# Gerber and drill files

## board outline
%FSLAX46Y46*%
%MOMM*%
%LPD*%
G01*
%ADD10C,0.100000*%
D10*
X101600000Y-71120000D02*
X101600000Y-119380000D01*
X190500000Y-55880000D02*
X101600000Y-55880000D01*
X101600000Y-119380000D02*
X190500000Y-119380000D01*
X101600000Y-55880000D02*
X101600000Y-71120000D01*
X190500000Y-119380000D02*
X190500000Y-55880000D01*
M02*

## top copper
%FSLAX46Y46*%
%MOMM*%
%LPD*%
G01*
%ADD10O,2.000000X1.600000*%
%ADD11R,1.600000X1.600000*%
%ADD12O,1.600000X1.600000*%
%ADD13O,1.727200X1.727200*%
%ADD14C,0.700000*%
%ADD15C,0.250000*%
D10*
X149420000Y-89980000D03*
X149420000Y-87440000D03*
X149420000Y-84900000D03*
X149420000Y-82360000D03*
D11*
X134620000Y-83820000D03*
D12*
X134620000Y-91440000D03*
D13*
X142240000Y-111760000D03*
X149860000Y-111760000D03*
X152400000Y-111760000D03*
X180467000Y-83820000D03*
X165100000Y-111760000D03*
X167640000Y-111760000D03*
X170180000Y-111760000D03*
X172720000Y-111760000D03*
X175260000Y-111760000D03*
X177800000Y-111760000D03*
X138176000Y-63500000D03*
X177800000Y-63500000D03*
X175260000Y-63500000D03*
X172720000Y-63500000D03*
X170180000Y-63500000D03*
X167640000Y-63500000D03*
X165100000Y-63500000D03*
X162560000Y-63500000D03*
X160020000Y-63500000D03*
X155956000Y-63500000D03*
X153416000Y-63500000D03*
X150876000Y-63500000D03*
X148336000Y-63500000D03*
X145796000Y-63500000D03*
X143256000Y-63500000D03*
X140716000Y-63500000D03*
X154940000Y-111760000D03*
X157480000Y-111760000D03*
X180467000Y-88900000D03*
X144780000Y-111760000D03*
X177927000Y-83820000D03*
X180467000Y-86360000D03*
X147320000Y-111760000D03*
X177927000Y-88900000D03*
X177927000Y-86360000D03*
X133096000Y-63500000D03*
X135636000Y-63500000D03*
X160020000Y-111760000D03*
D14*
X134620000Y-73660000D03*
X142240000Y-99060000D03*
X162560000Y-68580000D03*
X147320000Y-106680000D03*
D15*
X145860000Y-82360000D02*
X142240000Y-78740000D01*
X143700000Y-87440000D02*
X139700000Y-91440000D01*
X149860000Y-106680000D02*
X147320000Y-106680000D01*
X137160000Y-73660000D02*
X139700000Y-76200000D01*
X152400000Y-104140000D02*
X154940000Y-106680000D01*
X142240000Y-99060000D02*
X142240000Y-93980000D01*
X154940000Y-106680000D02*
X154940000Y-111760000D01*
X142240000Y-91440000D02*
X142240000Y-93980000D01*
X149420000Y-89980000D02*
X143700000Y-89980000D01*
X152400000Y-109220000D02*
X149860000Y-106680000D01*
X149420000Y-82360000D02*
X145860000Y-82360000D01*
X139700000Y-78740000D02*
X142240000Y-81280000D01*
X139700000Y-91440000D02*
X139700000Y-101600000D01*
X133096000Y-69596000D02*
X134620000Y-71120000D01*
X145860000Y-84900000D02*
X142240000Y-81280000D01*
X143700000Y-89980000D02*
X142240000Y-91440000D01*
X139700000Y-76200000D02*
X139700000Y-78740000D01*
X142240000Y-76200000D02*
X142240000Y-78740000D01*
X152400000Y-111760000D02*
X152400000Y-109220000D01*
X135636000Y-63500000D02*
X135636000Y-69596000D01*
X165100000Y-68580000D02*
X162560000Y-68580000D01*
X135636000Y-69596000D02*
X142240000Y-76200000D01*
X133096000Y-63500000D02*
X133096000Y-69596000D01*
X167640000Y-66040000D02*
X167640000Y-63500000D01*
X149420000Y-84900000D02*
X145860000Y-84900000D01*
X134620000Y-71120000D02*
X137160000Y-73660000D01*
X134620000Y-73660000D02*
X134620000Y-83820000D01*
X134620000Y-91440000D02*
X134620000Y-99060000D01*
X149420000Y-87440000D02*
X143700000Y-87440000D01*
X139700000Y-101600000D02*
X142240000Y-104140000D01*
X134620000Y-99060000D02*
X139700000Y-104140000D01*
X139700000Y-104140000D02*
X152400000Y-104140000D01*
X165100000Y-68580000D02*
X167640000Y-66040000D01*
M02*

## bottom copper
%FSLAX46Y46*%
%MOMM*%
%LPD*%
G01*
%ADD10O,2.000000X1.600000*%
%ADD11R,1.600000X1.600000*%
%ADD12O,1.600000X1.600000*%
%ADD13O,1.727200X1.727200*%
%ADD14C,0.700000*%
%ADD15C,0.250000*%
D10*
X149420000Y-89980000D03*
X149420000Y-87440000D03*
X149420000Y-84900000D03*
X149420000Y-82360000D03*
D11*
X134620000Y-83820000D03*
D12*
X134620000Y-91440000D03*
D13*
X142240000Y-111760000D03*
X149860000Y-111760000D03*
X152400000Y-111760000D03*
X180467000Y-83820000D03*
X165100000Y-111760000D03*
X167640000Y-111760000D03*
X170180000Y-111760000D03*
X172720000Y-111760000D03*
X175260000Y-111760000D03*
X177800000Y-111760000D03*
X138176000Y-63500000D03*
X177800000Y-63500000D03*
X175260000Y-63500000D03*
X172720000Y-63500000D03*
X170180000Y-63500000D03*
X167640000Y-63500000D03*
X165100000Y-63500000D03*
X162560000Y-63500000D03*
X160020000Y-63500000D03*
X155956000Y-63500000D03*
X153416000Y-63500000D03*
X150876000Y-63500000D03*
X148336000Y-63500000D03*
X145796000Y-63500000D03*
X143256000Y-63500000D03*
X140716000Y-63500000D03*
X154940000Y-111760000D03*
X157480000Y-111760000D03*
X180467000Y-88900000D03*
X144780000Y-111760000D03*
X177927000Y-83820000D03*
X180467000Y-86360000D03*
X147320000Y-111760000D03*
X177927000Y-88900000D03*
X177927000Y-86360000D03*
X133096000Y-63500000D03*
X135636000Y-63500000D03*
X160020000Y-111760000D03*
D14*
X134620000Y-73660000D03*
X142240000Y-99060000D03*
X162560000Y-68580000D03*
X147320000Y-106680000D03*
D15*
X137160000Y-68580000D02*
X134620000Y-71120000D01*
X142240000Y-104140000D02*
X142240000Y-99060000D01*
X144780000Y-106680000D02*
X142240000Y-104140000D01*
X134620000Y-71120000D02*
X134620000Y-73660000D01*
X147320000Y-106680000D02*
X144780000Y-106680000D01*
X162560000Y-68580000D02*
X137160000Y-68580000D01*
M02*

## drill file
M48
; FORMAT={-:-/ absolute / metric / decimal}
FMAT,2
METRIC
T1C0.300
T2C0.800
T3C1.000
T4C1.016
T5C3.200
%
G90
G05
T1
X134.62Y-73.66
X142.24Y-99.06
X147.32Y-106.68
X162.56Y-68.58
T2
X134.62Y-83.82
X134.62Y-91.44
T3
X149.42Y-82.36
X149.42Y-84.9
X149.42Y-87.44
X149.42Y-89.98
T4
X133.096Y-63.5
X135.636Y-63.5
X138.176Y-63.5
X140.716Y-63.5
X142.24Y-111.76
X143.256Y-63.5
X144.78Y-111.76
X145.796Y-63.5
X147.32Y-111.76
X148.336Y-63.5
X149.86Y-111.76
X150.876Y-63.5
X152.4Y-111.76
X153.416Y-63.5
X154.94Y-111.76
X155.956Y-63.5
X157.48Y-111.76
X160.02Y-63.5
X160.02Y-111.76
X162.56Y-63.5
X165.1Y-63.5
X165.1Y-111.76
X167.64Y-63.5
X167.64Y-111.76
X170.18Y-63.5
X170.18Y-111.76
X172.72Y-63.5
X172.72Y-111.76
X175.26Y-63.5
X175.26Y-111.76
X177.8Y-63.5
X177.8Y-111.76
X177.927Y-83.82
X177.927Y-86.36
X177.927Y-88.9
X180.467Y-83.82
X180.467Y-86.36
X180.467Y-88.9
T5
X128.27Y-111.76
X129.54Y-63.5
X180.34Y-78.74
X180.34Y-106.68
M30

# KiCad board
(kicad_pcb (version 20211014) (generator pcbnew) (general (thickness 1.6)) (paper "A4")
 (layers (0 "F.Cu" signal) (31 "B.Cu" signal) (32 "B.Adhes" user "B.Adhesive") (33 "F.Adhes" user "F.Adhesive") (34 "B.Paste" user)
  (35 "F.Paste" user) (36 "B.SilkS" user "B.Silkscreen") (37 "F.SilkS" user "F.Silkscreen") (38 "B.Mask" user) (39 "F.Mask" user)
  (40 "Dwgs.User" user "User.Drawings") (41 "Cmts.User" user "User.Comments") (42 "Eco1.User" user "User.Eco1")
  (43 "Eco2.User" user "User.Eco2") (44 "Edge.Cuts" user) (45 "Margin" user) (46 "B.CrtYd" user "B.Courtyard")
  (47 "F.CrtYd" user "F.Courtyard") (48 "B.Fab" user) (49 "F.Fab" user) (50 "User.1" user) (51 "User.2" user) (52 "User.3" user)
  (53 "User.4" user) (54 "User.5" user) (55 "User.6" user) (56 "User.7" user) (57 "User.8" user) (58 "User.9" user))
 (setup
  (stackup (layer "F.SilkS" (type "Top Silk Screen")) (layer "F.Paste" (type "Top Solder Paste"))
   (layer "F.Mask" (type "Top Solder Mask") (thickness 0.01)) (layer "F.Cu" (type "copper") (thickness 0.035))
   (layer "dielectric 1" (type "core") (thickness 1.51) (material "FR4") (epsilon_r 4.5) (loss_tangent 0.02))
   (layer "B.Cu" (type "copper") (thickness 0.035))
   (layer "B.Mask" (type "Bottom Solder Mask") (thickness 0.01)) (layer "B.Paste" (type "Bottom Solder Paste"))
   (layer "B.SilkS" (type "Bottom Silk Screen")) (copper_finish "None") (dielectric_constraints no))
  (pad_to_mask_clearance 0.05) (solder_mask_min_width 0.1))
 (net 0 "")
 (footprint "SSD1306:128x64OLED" (layer "F.Cu") (at 160.02 86.36 90)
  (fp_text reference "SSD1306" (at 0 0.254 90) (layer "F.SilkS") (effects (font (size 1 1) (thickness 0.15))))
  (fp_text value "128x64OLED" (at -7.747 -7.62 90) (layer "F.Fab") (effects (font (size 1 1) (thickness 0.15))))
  (pad "1" thru_hole oval locked (at -3.62 -10.6 180) (size 2 1.6) (drill 1) (layers *.Cu *.Mask))
  (pad "2" thru_hole oval locked (at -1.08 -10.6 180) (size 2 1.6) (drill 1) (layers *.Cu *.Mask))
  (pad "3" thru_hole oval locked (at 1.46 -10.6 180) (size 2 1.6) (drill 1) (layers *.Cu *.Mask))
  (pad "4" thru_hole oval locked (at 4 -10.6 180) (size 2 1.6) (drill 1) (layers *.Cu *.Mask)))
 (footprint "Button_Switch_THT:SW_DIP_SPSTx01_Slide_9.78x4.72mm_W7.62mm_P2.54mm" (layer "F.Cu") (at 134.62 83.82 -90)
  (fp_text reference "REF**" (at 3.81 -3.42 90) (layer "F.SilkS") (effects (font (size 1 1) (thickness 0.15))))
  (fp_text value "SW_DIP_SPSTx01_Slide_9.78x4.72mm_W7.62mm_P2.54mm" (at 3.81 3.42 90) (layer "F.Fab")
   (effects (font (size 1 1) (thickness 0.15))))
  (pad "1" thru_hole rect (at 0 0 270) (size 1.6 1.6) (drill 0.8) (layers *.Cu *.Mask))
  (pad "2" thru_hole oval (at 7.62 0 270) (size 1.6 1.6) (drill 0.8) (layers *.Cu *.Mask)))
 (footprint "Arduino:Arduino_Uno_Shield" (layer "F.Cu") (at 114.3 114.3)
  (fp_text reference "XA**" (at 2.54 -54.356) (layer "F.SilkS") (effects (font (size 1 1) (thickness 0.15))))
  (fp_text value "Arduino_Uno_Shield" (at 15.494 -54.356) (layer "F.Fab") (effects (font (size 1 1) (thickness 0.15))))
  (pad "" np_thru_hole circle (at 66.04 -35.56) (size 3.2 3.2) (drill 3.2) (layers *.Cu *.Mask))
  (pad "" np_thru_hole circle (at 66.04 -7.62) (size 3.2 3.2) (drill 3.2) (layers *.Cu *.Mask))
  (pad "" np_thru_hole circle (at 13.97 -2.54) (size 3.2 3.2) (drill 3.2) (layers *.Cu *.Mask))
  (pad "" thru_hole oval (at 27.94 -2.54) (size 1.7272 1.7272) (drill 1.016) (layers *.Cu *.Mask))
  (pad "" np_thru_hole circle (at 15.24 -50.8) (size 3.2 3.2) (drill 3.2) (layers *.Cu *.Mask))
  (pad "3V3" thru_hole oval (at 35.56 -2.54) (size 1.7272 1.7272) (drill 1.016) (layers *.Cu *.Mask))
  (pad "5V1" thru_hole oval (at 38.1 -2.54) (size 1.7272 1.7272) (drill 1.016) (layers *.Cu *.Mask))
  (pad "5V2" thru_hole oval (at 66.167 -30.48) (size 1.7272 1.7272) (drill 1.016) (layers *.Cu *.Mask))
  (pad "A0" thru_hole oval (at 50.8 -2.54) (size 1.7272 1.7272) (drill 1.016) (layers *.Cu *.Mask))
  (pad "A1" thru_hole oval (at 53.34 -2.54) (size 1.7272 1.7272) (drill 1.016) (layers *.Cu *.Mask))
  (pad "A2" thru_hole oval (at 55.88 -2.54) (size 1.7272 1.7272) (drill 1.016) (layers *.Cu *.Mask))
  (pad "A3" thru_hole oval (at 58.42 -2.54) (size 1.7272 1.7272) (drill 1.016) (layers *.Cu *.Mask))
  (pad "A4" thru_hole oval (at 60.96 -2.54) (size 1.7272 1.7272) (drill 1.016) (layers *.Cu *.Mask))
  (pad "A5" thru_hole oval (at 63.5 -2.54) (size 1.7272 1.7272) (drill 1.016) (layers *.Cu *.Mask))
  (pad "AREF" thru_hole oval (at 23.876 -50.8) (size 1.7272 1.7272) (drill 1.016) (layers *.Cu *.Mask))
  (pad "D0" thru_hole oval (at 63.5 -50.8) (size 1.7272 1.7272) (drill 1.016) (layers *.Cu *.Mask))
  (pad "D1" thru_hole oval (at 60.96 -50.8) (size 1.7272 1.7272) (drill 1.016) (layers *.Cu *.Mask))
  (pad "D2" thru_hole oval (at 58.42 -50.8) (size 1.7272 1.7272) (drill 1.016) (layers *.Cu *.Mask))
  (pad "D3" thru_hole oval (at 55.88 -50.8) (size 1.7272 1.7272) (drill 1.016) (layers *.Cu *.Mask))
  (pad "D4" thru_hole oval (at 53.34 -50.8) (size 1.7272 1.7272) (drill 1.016) (layers *.Cu *.Mask))
  (pad "D5" thru_hole oval (at 50.8 -50.8) (size 1.7272 1.7272) (drill 1.016) (layers *.Cu *.Mask))
  (pad "D6" thru_hole oval (at 48.26 -50.8) (size 1.7272 1.7272) (drill 1.016) (layers *.Cu *.Mask))
  (pad "D7" thru_hole oval (at 45.72 -50.8) (size 1.7272 1.7272) (drill 1.016) (layers *.Cu *.Mask))
  (pad "D8" thru_hole oval (at 41.656 -50.8) (size 1.7272 1.7272) (drill 1.016) (layers *.Cu *.Mask))
  (pad "D9" thru_hole oval (at 39.116 -50.8) (size 1.7272 1.7272) (drill 1.016) (layers *.Cu *.Mask))
  (pad "D10" thru_hole oval (at 36.576 -50.8) (size 1.7272 1.7272) (drill 1.016) (layers *.Cu *.Mask))
  (pad "D11" thru_hole oval (at 34.036 -50.8) (size 1.7272 1.7272) (drill 1.016) (layers *.Cu *.Mask))
  (pad "D12" thru_hole oval (at 31.496 -50.8) (size 1.7272 1.7272) (drill 1.016) (layers *.Cu *.Mask))
  (pad "D13" thru_hole oval (at 28.956 -50.8) (size 1.7272 1.7272) (drill 1.016) (layers *.Cu *.Mask))
  (pad "GND1" thru_hole oval (at 26.416 -50.8) (size 1.7272 1.7272) (drill 1.016) (layers *.Cu *.Mask))
  (pad "GND2" thru_hole oval (at 40.64 -2.54) (size 1.7272 1.7272) (drill 1.016) (layers *.Cu *.Mask))
  (pad "GND3" thru_hole oval (at 43.18 -2.54) (size 1.7272 1.7272) (drill 1.016) (layers *.Cu *.Mask))
  (pad "GND4" thru_hole oval (at 66.167 -25.4) (size 1.7272 1.7272) (drill 1.016) (layers *.Cu *.Mask))
  (pad "IORF" thru_hole oval (at 30.48 -2.54) (size 1.7272 1.7272) (drill 1.016) (layers *.Cu *.Mask))
  (pad "MISO" thru_hole oval (at 63.627 -30.48) (size 1.7272 1.7272) (drill 1.016) (layers *.Cu *.Mask))
  (pad "MOSI" thru_hole oval (at 66.167 -27.94) (size 1.7272 1.7272) (drill 1.016) (layers *.Cu *.Mask))
  (pad "RST1" thru_hole oval (at 33.02 -2.54) (size 1.7272 1.7272) (drill 1.016) (layers *.Cu *.Mask))
  (pad "RST2" thru_hole oval (at 63.627 -25.4) (size 1.7272 1.7272) (drill 1.016) (layers *.Cu *.Mask))
  (pad "SCK" thru_hole oval (at 63.627 -27.94) (size 1.7272 1.7272) (drill 1.016) (layers *.Cu *.Mask))
  (pad "SCL" thru_hole oval (at 18.796 -50.8) (size 1.7272 1.7272) (drill 1.016) (layers *.Cu *.Mask))
  (pad "SDA" thru_hole oval (at 21.336 -50.8) (size 1.7272 1.7272) (drill 1.016) (layers *.Cu *.Mask))
  (pad "VIN" thru_hole oval (at 45.72 -2.54) (size 1.7272 1.7272) (drill 1.016) (layers *.Cu *.Mask)))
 (gr_line (start 101.6 71.12) (end 101.6 119.38) (layer "Edge.Cuts") (width 0.1))
 (gr_line (start 190.5 55.88) (end 101.6 55.88) (layer "Edge.Cuts") (width 0.1))
 (gr_line (start 101.6 119.38) (end 190.5 119.38) (layer "Edge.Cuts") (width 0.1))
 (gr_line (start 101.6 55.88) (end 101.6 71.12) (layer "Edge.Cuts") (width 0.1))
 (gr_line (start 190.5 119.38) (end 190.5 55.88) (layer "Edge.Cuts") (width 0.1))
 (segment (start 145.86 82.36) (end 142.24 78.74) (width 0.25) (layer "F.Cu") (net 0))
 (segment (start 143.7 87.44) (end 139.7 91.44) (width 0.25) (layer "F.Cu") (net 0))
 (segment (start 149.86 106.68) (end 147.32 106.68) (width 0.25) (layer "F.Cu") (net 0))
 (segment (start 137.16 73.66) (end 139.7 76.2) (width 0.25) (layer "F.Cu") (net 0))
 (segment (start 152.4 104.14) (end 154.94 106.68) (width 0.25) (layer "F.Cu") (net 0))
 (segment (start 142.24 99.06) (end 142.24 93.98) (width 0.25) (layer "F.Cu") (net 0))
 (segment (start 154.94 106.68) (end 154.94 111.76) (width 0.25) (layer "F.Cu") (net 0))
 (segment (start 142.24 91.44) (end 142.24 93.98) (width 0.25) (layer "F.Cu") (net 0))
 (segment (start 149.42 89.98) (end 143.7 89.98) (width 0.25) (layer "F.Cu") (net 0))
 (segment (start 152.4 109.22) (end 149.86 106.68) (width 0.25) (layer "F.Cu") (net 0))
 (segment (start 149.42 82.36) (end 145.86 82.36) (width 0.25) (layer "F.Cu") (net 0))
 (segment (start 139.7 78.74) (end 142.24 81.28) (width 0.25) (layer "F.Cu") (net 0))
 (segment (start 139.7 91.44) (end 139.7 101.6) (width 0.25) (layer "F.Cu") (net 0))
 (segment (start 133.096 69.596) (end 134.62 71.12) (width 0.25) (layer "F.Cu") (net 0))
 (segment (start 145.86 84.9) (end 142.24 81.28) (width 0.25) (layer "F.Cu") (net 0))
 (segment (start 143.7 89.98) (end 142.24 91.44) (width 0.25) (layer "F.Cu") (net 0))
 (segment (start 139.7 76.2) (end 139.7 78.74) (width 0.25) (layer "F.Cu") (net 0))
 (segment (start 142.24 76.2) (end 142.24 78.74) (width 0.25) (layer "F.Cu") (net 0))
 (segment (start 152.4 111.76) (end 152.4 109.22) (width 0.25) (layer "F.Cu") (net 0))
 (segment (start 135.636 63.5) (end 135.636 69.596) (width 0.25) (layer "F.Cu") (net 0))
 (segment (start 165.1 68.58) (end 162.56 68.58) (width 0.25) (layer "F.Cu") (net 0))
 (segment (start 135.636 69.596) (end 142.24 76.2) (width 0.25) (layer "F.Cu") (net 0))
 (segment (start 133.096 63.5) (end 133.096 69.596) (width 0.25) (layer "F.Cu") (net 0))
 (segment (start 167.64 66.04) (end 167.64 63.5) (width 0.25) (layer "F.Cu") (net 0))
 (segment (start 149.42 84.9) (end 145.86 84.9) (width 0.25) (layer "F.Cu") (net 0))
 (segment (start 134.62 71.12) (end 137.16 73.66) (width 0.25) (layer "F.Cu") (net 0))
 (segment (start 134.62 73.66) (end 134.62 83.82) (width 0.25) (layer "F.Cu") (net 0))
 (segment (start 134.62 91.44) (end 134.62 99.06) (width 0.25) (layer "F.Cu") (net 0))
 (segment (start 149.42 87.44) (end 143.7 87.44) (width 0.25) (layer "F.Cu") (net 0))
 (segment (start 139.7 101.6) (end 142.24 104.14) (width 0.25) (layer "F.Cu") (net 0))
 (segment (start 134.62 99.06) (end 139.7 104.14) (width 0.25) (layer "F.Cu") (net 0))
 (segment (start 139.7 104.14) (end 152.4 104.14) (width 0.25) (layer "F.Cu") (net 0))
 (segment (start 165.1 68.58) (end 167.64 66.04) (width 0.25) (layer "F.Cu") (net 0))
 (via (at 134.62 73.66) (size 0.7) (drill 0.3) (layers "F.Cu" "B.Cu") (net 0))
 (via (at 142.24 99.06) (size 0.7) (drill 0.3) (layers "F.Cu" "B.Cu") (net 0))
 (via (at 162.56 68.58) (size 0.7) (drill 0.3) (layers "F.Cu" "B.Cu") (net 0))
 (via (at 147.32 106.68) (size 0.7) (drill 0.3) (layers "F.Cu" "B.Cu") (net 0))
 (segment (start 137.16 68.58) (end 134.62 71.12) (width 0.25) (layer "B.Cu") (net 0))
 (segment (start 142.24 104.14) (end 142.24 99.06) (width 0.25) (layer "B.Cu") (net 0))
 (segment (start 144.78 106.68) (end 142.24 104.14) (width 0.25) (layer "B.Cu") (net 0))
 (segment (start 134.62 71.12) (end 134.62 73.66) (width 0.25) (layer "B.Cu") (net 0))
 (segment (start 147.32 106.68) (end 144.78 106.68) (width 0.25) (layer "B.Cu") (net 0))
 (segment (start 162.56 68.58) (end 137.16 68.58) (width 0.25) (layer "B.Cu") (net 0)))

